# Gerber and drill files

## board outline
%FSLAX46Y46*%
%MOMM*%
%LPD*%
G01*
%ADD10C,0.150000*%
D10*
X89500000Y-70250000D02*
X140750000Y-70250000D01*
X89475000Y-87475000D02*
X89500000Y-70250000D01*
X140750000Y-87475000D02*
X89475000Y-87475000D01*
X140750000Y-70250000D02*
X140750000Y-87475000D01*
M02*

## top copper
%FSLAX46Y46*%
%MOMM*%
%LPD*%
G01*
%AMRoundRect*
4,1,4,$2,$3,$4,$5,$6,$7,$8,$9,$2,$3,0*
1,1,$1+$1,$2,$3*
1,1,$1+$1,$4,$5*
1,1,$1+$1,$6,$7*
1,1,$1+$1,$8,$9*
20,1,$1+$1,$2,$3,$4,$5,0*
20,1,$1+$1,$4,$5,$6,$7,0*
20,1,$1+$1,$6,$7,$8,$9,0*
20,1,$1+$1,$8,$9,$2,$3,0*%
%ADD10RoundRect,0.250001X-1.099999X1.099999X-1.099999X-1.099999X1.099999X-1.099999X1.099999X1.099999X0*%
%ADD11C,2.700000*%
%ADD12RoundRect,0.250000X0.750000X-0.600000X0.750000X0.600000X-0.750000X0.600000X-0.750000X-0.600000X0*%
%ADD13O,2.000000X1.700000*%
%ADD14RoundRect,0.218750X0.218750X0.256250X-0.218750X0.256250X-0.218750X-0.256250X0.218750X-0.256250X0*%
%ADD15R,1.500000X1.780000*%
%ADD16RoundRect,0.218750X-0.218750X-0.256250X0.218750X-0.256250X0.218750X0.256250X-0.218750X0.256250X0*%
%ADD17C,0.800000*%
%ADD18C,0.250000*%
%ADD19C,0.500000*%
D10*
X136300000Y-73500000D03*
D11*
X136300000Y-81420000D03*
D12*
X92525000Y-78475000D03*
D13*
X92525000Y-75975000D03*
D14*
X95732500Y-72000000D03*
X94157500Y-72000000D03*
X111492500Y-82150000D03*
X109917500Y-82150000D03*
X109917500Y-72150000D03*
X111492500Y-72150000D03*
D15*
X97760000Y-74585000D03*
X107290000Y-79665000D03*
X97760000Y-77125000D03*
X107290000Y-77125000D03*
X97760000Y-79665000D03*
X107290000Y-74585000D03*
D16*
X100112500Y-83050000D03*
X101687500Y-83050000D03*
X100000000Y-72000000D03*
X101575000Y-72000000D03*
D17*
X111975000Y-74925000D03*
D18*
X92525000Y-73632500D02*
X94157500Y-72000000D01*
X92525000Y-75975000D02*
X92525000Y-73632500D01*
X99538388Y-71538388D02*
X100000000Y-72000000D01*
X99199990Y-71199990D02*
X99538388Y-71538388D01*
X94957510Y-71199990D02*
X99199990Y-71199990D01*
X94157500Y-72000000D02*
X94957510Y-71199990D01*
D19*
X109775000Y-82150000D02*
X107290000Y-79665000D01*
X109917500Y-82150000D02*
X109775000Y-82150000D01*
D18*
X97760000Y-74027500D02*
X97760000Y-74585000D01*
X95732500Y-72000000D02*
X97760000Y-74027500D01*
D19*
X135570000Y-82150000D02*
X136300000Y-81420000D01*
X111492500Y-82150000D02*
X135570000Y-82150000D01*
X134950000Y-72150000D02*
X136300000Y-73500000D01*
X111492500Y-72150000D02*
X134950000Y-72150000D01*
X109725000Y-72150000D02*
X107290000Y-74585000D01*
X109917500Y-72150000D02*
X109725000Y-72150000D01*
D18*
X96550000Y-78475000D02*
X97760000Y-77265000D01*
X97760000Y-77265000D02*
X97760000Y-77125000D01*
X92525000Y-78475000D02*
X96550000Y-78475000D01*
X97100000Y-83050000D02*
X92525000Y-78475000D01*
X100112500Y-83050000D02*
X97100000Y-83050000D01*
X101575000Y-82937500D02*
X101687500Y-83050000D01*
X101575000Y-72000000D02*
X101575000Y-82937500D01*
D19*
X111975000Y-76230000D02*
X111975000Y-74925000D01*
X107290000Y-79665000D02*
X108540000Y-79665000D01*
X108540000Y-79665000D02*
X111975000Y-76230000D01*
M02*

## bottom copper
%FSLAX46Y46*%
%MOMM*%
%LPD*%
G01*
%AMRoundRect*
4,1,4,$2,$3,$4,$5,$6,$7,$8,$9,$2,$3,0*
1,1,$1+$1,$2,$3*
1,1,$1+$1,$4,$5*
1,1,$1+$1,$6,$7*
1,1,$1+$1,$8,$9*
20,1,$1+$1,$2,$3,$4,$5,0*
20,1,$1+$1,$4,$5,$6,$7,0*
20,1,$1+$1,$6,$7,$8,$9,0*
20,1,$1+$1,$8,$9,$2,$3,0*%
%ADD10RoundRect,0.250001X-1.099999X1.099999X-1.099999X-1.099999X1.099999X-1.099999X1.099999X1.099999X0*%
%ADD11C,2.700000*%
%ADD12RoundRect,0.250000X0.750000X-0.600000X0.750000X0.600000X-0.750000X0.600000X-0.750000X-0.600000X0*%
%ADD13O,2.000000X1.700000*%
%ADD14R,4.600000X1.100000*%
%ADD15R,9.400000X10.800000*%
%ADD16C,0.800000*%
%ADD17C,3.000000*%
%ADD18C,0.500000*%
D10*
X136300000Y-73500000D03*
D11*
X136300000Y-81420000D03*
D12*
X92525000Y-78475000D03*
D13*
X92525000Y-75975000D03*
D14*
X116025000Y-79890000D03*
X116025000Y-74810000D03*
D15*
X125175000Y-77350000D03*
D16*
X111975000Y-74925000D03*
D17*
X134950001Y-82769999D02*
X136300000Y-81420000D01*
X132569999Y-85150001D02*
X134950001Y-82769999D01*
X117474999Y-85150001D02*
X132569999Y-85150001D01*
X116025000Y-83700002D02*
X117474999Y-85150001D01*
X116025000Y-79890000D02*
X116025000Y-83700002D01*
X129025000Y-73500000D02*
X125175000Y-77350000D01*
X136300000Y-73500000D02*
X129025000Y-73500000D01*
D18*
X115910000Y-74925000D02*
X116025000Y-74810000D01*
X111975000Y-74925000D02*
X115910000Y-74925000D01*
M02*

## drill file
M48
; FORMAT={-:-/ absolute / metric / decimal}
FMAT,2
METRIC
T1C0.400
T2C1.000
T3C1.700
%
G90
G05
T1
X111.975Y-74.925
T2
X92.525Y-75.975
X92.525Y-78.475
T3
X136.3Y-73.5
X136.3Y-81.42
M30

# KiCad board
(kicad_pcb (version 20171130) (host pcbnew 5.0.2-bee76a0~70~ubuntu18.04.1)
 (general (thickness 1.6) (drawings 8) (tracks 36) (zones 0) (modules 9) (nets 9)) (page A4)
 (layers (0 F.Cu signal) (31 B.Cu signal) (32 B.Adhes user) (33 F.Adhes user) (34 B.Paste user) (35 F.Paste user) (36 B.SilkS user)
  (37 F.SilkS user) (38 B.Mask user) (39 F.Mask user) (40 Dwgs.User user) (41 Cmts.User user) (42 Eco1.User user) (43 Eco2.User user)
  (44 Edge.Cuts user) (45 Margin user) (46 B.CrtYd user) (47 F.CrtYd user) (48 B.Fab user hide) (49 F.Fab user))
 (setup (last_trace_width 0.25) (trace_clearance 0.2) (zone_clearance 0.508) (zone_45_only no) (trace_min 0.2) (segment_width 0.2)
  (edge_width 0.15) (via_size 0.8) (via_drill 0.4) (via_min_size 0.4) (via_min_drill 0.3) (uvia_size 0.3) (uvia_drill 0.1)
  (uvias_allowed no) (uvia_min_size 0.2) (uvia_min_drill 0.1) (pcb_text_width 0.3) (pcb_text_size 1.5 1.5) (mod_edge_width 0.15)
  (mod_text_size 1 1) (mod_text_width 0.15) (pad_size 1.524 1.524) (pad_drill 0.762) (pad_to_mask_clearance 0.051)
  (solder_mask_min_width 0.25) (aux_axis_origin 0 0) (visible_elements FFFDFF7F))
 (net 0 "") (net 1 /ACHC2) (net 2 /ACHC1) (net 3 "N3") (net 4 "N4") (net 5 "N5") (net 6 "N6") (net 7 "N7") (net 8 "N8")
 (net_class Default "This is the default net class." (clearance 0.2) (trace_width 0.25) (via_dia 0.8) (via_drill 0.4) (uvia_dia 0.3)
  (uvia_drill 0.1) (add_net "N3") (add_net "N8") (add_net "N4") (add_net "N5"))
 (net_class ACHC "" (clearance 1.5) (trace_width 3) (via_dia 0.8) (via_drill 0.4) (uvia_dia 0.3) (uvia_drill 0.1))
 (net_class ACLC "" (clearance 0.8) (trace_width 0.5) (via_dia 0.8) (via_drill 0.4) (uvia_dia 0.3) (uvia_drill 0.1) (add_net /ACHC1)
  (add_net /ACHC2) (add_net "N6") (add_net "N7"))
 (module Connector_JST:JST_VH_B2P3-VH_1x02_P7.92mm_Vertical (layer F.Cu) (at 136.3 73.5 270)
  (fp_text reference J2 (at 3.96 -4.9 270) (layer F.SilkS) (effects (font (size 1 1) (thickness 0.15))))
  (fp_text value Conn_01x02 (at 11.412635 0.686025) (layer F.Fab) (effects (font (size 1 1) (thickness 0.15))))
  (pad 1 thru_hole roundrect (at 0 0 270) (size 2.7 2.7) (drill 1.7) (layers *.Cu *.Mask) (roundrect_rratio 0.09259299999999999)
   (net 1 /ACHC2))
  (pad 2 thru_hole circle (at 7.92 0 270) (size 2.7 2.7) (drill 1.7) (layers *.Cu *.Mask) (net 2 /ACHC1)))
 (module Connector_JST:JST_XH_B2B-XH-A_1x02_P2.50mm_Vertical (layer F.Cu) (at 92.525 78.475 90)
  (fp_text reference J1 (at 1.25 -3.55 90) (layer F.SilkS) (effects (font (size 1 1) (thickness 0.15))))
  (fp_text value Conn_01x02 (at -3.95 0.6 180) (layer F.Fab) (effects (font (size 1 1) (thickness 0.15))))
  (pad 1 thru_hole roundrect (at 0 0 90) (size 1.7 2) (drill 1) (layers *.Cu *.Mask) (roundrect_rratio 0.147059) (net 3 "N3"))
  (pad 2 thru_hole oval (at 2.5 0 90) (size 1.7 2) (drill 1) (layers *.Cu *.Mask) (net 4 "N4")))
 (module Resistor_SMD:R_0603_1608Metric (layer F.Cu) (at 94.945 72 180)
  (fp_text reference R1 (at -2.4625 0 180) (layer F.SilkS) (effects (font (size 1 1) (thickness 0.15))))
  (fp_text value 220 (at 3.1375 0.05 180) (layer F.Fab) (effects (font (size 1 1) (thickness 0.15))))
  (pad 1 smd roundrect (at -0.7875 0 180) (size 0.875 0.95) (layers F.Cu F.Paste F.Mask) (roundrect_rratio 0.25) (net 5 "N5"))
  (pad 2 smd roundrect (at 0.7875 0 180) (size 0.875 0.95) (layers F.Cu F.Paste F.Mask) (roundrect_rratio 0.25) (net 4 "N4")))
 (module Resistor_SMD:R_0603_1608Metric (layer F.Cu) (at 110.705 82.15 180)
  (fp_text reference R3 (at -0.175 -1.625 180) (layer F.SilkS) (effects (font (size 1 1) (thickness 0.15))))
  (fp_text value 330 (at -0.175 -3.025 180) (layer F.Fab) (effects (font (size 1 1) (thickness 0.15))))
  (pad 1 smd roundrect (at -0.7875 0 180) (size 0.875 0.95) (layers F.Cu F.Paste F.Mask) (roundrect_rratio 0.25) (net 2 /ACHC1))
  (pad 2 smd roundrect (at 0.7875 0 180) (size 0.875 0.95) (layers F.Cu F.Paste F.Mask) (roundrect_rratio 0.25) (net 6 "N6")))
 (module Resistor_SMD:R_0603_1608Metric (layer F.Cu) (at 110.705 72.15 180)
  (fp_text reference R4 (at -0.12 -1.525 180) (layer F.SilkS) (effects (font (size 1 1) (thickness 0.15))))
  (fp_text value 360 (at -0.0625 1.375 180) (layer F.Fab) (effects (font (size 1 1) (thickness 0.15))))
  (pad 2 smd roundrect (at 0.7875 0 180) (size 0.875 0.95) (layers F.Cu F.Paste F.Mask) (roundrect_rratio 0.25) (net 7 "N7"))
  (pad 1 smd roundrect (at -0.7875 0 180) (size 0.875 0.95) (layers F.Cu F.Paste F.Mask) (roundrect_rratio 0.25) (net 1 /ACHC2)))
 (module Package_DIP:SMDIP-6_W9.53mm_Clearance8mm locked (layer F.Cu) (at 102.525 77.125)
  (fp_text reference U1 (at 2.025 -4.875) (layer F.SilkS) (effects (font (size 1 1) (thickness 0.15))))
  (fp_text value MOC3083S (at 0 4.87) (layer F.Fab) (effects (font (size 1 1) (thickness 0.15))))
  (pad 1 smd rect (at -4.765 -2.54) (size 1.5 1.78) (layers F.Cu F.Paste F.Mask) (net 5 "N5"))
  (pad 4 smd rect (at 4.765 2.54) (size 1.5 1.78) (layers F.Cu F.Paste F.Mask) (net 6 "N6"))
  (pad 2 smd rect (at -4.765 0) (size 1.5 1.78) (layers F.Cu F.Paste F.Mask) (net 3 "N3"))
  (pad 5 smd rect (at 4.765 0) (size 1.5 1.78) (layers F.Cu F.Paste F.Mask))
  (pad 3 smd rect (at -4.765 2.54) (size 1.5 1.78) (layers F.Cu F.Paste F.Mask))
  (pad 6 smd rect (at 4.765 -2.54) (size 1.5 1.78) (layers F.Cu F.Paste F.Mask) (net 7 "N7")))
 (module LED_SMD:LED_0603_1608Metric (layer F.Cu) (at 100.9 83.05)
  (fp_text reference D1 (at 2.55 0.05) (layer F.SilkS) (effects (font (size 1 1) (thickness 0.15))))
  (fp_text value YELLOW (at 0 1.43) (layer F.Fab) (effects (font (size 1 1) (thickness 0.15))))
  (pad 1 smd roundrect (at -0.7875 0) (size 0.875 0.95) (layers F.Cu F.Paste F.Mask) (roundrect_rratio 0.25) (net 3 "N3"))
  (pad 2 smd roundrect (at 0.7875 0) (size 0.875 0.95) (layers F.Cu F.Paste F.Mask) (roundrect_rratio 0.25) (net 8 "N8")))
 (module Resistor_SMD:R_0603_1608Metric (layer F.Cu) (at 100.7875 72)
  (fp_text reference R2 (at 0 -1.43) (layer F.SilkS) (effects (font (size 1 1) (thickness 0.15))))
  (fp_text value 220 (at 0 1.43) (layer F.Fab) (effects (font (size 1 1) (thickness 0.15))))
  (pad 1 smd roundrect (at -0.7875 0) (size 0.875 0.95) (layers F.Cu F.Paste F.Mask) (roundrect_rratio 0.25) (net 4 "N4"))
  (pad 2 smd roundrect (at 0.7875 0) (size 0.875 0.95) (layers F.Cu F.Paste F.Mask) (roundrect_rratio 0.25) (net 8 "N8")))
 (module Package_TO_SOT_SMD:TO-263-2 (layer B.Cu) (at 121.8 77.35)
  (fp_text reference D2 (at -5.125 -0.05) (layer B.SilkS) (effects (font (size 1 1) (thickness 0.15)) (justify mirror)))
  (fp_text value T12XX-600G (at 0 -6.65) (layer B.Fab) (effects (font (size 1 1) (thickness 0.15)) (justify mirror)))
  (pad 1 smd rect (at -5.775 2.54) (size 4.6 1.1) (layers B.Cu B.Paste B.Mask) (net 2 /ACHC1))
  (pad 3 smd rect (at -5.775 -2.54) (size 4.6 1.1) (layers B.Cu B.Paste B.Mask) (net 6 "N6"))
  (pad 2 smd rect (at 3.375 0) (size 9.4 10.8) (layers B.Cu B.Mask) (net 1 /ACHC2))
  (pad "" smd rect (at 5.8 -2.775) (size 4.55 5.25) (layers B.Paste))
  (pad "" smd rect (at 0.95 2.775) (size 4.55 5.25) (layers B.Paste))
  (pad "" smd rect (at 5.8 2.775) (size 4.55 5.25) (layers B.Paste))
  (pad "" smd rect (at 0.95 -2.775) (size 4.55 5.25) (layers B.Paste)))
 (gr_line (start 89.5 70.25) (end 140.75 70.25) (layer Edge.Cuts) (width 0.15))
 (gr_line (start 89.475 87.475) (end 89.5 70.25) (layer Edge.Cuts) (width 0.15))
 (gr_line (start 140.75 87.475) (end 89.475 87.475) (layer Edge.Cuts) (width 0.15))
 (gr_line (start 140.75 70.25) (end 140.75 87.475) (layer Edge.Cuts) (width 0.15))
 (segment (start 92.525 73.6325) (end 94.1575 72) (width 0.25) (layer F.Cu) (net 4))
 (segment (start 92.525 75.975) (end 92.525 73.6325) (width 0.25) (layer F.Cu) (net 4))
 (segment (start 99.538388 71.538388) (end 100 72) (width 0.25) (layer F.Cu) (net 4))
 (segment (start 99.19999 71.19999) (end 99.538388 71.538388) (width 0.25) (layer F.Cu) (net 4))
 (segment (start 94.95751 71.19999) (end 99.19999 71.19999) (width 0.25) (layer F.Cu) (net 4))
 (segment (start 94.1575 72) (end 94.95751 71.19999) (width 0.25) (layer F.Cu) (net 4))
 (segment (start 109.775 82.15) (end 107.29 79.665) (width 0.5) (layer F.Cu) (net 6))
 (segment (start 109.9175 82.15) (end 109.775 82.15) (width 0.5) (layer F.Cu) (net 6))
 (segment (start 97.76 74.0275) (end 97.76 74.585) (width 0.25) (layer F.Cu) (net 5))
 (segment (start 95.7325 72) (end 97.76 74.0275) (width 0.25) (layer F.Cu) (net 5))
 (segment (start 134.950001 82.769999) (end 136.3 81.42) (width 3) (layer B.Cu) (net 2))
 (segment (start 132.569999 85.150001) (end 134.950001 82.769999) (width 3) (layer B.Cu) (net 2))
 (segment (start 117.474999 85.150001) (end 132.569999 85.150001) (width 3) (layer B.Cu) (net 2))
 (segment (start 116.025 83.700002) (end 117.474999 85.150001) (width 3) (layer B.Cu) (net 2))
 (segment (start 116.025 79.89) (end 116.025 83.700002) (width 3) (layer B.Cu) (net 2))
 (segment (start 135.57 82.15) (end 136.3 81.42) (width 0.5) (layer F.Cu) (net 2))
 (segment (start 111.4925 82.15) (end 135.57 82.15) (width 0.5) (layer F.Cu) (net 2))
 (segment (start 129.025 73.5) (end 125.175 77.35) (width 3) (layer B.Cu) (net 1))
 (segment (start 136.3 73.5) (end 129.025 73.5) (width 3) (layer B.Cu) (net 1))
 (segment (start 134.95 72.15) (end 136.3 73.5) (width 0.5) (layer F.Cu) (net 1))
 (segment (start 111.4925 72.15) (end 134.95 72.15) (width 0.5) (layer F.Cu) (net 1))
 (segment (start 109.725 72.15) (end 107.29 74.585) (width 0.5) (layer F.Cu) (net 7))
 (segment (start 109.9175 72.15) (end 109.725 72.15) (width 0.5) (layer F.Cu) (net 7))
 (segment (start 96.55 78.475) (end 97.76 77.265) (width 0.25) (layer F.Cu) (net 3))
 (segment (start 97.76 77.265) (end 97.76 77.125) (width 0.25) (layer F.Cu) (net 3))
 (segment (start 92.525 78.475) (end 96.55 78.475) (width 0.25) (layer F.Cu) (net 3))
 (segment (start 97.1 83.05) (end 92.525 78.475) (width 0.25) (layer F.Cu) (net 3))
 (segment (start 100.1125 83.05) (end 97.1 83.05) (width 0.25) (layer F.Cu) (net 3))
 (segment (start 101.575 82.9375) (end 101.6875 83.05) (width 0.25) (layer F.Cu) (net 8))
 (segment (start 101.575 72) (end 101.575 82.9375) (width 0.25) (layer F.Cu) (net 8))
 (segment (start 111.975 76.23) (end 111.975 74.925) (width 0.5) (layer F.Cu) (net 6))
 (segment (start 107.29 79.665) (end 108.54 79.665) (width 0.5) (layer F.Cu) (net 6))
 (via (at 111.975 74.925) (size 0.8) (drill 0.4) (layers F.Cu B.Cu) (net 6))
 (segment (start 108.54 79.665) (end 111.975 76.23) (width 0.5) (layer F.Cu) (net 6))
 (segment (start 115.91 74.925) (end 116.025 74.81) (width 0.5) (layer B.Cu) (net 6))
 (segment (start 111.975 74.925) (end 115.91 74.925) (width 0.5) (layer B.Cu) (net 6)))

